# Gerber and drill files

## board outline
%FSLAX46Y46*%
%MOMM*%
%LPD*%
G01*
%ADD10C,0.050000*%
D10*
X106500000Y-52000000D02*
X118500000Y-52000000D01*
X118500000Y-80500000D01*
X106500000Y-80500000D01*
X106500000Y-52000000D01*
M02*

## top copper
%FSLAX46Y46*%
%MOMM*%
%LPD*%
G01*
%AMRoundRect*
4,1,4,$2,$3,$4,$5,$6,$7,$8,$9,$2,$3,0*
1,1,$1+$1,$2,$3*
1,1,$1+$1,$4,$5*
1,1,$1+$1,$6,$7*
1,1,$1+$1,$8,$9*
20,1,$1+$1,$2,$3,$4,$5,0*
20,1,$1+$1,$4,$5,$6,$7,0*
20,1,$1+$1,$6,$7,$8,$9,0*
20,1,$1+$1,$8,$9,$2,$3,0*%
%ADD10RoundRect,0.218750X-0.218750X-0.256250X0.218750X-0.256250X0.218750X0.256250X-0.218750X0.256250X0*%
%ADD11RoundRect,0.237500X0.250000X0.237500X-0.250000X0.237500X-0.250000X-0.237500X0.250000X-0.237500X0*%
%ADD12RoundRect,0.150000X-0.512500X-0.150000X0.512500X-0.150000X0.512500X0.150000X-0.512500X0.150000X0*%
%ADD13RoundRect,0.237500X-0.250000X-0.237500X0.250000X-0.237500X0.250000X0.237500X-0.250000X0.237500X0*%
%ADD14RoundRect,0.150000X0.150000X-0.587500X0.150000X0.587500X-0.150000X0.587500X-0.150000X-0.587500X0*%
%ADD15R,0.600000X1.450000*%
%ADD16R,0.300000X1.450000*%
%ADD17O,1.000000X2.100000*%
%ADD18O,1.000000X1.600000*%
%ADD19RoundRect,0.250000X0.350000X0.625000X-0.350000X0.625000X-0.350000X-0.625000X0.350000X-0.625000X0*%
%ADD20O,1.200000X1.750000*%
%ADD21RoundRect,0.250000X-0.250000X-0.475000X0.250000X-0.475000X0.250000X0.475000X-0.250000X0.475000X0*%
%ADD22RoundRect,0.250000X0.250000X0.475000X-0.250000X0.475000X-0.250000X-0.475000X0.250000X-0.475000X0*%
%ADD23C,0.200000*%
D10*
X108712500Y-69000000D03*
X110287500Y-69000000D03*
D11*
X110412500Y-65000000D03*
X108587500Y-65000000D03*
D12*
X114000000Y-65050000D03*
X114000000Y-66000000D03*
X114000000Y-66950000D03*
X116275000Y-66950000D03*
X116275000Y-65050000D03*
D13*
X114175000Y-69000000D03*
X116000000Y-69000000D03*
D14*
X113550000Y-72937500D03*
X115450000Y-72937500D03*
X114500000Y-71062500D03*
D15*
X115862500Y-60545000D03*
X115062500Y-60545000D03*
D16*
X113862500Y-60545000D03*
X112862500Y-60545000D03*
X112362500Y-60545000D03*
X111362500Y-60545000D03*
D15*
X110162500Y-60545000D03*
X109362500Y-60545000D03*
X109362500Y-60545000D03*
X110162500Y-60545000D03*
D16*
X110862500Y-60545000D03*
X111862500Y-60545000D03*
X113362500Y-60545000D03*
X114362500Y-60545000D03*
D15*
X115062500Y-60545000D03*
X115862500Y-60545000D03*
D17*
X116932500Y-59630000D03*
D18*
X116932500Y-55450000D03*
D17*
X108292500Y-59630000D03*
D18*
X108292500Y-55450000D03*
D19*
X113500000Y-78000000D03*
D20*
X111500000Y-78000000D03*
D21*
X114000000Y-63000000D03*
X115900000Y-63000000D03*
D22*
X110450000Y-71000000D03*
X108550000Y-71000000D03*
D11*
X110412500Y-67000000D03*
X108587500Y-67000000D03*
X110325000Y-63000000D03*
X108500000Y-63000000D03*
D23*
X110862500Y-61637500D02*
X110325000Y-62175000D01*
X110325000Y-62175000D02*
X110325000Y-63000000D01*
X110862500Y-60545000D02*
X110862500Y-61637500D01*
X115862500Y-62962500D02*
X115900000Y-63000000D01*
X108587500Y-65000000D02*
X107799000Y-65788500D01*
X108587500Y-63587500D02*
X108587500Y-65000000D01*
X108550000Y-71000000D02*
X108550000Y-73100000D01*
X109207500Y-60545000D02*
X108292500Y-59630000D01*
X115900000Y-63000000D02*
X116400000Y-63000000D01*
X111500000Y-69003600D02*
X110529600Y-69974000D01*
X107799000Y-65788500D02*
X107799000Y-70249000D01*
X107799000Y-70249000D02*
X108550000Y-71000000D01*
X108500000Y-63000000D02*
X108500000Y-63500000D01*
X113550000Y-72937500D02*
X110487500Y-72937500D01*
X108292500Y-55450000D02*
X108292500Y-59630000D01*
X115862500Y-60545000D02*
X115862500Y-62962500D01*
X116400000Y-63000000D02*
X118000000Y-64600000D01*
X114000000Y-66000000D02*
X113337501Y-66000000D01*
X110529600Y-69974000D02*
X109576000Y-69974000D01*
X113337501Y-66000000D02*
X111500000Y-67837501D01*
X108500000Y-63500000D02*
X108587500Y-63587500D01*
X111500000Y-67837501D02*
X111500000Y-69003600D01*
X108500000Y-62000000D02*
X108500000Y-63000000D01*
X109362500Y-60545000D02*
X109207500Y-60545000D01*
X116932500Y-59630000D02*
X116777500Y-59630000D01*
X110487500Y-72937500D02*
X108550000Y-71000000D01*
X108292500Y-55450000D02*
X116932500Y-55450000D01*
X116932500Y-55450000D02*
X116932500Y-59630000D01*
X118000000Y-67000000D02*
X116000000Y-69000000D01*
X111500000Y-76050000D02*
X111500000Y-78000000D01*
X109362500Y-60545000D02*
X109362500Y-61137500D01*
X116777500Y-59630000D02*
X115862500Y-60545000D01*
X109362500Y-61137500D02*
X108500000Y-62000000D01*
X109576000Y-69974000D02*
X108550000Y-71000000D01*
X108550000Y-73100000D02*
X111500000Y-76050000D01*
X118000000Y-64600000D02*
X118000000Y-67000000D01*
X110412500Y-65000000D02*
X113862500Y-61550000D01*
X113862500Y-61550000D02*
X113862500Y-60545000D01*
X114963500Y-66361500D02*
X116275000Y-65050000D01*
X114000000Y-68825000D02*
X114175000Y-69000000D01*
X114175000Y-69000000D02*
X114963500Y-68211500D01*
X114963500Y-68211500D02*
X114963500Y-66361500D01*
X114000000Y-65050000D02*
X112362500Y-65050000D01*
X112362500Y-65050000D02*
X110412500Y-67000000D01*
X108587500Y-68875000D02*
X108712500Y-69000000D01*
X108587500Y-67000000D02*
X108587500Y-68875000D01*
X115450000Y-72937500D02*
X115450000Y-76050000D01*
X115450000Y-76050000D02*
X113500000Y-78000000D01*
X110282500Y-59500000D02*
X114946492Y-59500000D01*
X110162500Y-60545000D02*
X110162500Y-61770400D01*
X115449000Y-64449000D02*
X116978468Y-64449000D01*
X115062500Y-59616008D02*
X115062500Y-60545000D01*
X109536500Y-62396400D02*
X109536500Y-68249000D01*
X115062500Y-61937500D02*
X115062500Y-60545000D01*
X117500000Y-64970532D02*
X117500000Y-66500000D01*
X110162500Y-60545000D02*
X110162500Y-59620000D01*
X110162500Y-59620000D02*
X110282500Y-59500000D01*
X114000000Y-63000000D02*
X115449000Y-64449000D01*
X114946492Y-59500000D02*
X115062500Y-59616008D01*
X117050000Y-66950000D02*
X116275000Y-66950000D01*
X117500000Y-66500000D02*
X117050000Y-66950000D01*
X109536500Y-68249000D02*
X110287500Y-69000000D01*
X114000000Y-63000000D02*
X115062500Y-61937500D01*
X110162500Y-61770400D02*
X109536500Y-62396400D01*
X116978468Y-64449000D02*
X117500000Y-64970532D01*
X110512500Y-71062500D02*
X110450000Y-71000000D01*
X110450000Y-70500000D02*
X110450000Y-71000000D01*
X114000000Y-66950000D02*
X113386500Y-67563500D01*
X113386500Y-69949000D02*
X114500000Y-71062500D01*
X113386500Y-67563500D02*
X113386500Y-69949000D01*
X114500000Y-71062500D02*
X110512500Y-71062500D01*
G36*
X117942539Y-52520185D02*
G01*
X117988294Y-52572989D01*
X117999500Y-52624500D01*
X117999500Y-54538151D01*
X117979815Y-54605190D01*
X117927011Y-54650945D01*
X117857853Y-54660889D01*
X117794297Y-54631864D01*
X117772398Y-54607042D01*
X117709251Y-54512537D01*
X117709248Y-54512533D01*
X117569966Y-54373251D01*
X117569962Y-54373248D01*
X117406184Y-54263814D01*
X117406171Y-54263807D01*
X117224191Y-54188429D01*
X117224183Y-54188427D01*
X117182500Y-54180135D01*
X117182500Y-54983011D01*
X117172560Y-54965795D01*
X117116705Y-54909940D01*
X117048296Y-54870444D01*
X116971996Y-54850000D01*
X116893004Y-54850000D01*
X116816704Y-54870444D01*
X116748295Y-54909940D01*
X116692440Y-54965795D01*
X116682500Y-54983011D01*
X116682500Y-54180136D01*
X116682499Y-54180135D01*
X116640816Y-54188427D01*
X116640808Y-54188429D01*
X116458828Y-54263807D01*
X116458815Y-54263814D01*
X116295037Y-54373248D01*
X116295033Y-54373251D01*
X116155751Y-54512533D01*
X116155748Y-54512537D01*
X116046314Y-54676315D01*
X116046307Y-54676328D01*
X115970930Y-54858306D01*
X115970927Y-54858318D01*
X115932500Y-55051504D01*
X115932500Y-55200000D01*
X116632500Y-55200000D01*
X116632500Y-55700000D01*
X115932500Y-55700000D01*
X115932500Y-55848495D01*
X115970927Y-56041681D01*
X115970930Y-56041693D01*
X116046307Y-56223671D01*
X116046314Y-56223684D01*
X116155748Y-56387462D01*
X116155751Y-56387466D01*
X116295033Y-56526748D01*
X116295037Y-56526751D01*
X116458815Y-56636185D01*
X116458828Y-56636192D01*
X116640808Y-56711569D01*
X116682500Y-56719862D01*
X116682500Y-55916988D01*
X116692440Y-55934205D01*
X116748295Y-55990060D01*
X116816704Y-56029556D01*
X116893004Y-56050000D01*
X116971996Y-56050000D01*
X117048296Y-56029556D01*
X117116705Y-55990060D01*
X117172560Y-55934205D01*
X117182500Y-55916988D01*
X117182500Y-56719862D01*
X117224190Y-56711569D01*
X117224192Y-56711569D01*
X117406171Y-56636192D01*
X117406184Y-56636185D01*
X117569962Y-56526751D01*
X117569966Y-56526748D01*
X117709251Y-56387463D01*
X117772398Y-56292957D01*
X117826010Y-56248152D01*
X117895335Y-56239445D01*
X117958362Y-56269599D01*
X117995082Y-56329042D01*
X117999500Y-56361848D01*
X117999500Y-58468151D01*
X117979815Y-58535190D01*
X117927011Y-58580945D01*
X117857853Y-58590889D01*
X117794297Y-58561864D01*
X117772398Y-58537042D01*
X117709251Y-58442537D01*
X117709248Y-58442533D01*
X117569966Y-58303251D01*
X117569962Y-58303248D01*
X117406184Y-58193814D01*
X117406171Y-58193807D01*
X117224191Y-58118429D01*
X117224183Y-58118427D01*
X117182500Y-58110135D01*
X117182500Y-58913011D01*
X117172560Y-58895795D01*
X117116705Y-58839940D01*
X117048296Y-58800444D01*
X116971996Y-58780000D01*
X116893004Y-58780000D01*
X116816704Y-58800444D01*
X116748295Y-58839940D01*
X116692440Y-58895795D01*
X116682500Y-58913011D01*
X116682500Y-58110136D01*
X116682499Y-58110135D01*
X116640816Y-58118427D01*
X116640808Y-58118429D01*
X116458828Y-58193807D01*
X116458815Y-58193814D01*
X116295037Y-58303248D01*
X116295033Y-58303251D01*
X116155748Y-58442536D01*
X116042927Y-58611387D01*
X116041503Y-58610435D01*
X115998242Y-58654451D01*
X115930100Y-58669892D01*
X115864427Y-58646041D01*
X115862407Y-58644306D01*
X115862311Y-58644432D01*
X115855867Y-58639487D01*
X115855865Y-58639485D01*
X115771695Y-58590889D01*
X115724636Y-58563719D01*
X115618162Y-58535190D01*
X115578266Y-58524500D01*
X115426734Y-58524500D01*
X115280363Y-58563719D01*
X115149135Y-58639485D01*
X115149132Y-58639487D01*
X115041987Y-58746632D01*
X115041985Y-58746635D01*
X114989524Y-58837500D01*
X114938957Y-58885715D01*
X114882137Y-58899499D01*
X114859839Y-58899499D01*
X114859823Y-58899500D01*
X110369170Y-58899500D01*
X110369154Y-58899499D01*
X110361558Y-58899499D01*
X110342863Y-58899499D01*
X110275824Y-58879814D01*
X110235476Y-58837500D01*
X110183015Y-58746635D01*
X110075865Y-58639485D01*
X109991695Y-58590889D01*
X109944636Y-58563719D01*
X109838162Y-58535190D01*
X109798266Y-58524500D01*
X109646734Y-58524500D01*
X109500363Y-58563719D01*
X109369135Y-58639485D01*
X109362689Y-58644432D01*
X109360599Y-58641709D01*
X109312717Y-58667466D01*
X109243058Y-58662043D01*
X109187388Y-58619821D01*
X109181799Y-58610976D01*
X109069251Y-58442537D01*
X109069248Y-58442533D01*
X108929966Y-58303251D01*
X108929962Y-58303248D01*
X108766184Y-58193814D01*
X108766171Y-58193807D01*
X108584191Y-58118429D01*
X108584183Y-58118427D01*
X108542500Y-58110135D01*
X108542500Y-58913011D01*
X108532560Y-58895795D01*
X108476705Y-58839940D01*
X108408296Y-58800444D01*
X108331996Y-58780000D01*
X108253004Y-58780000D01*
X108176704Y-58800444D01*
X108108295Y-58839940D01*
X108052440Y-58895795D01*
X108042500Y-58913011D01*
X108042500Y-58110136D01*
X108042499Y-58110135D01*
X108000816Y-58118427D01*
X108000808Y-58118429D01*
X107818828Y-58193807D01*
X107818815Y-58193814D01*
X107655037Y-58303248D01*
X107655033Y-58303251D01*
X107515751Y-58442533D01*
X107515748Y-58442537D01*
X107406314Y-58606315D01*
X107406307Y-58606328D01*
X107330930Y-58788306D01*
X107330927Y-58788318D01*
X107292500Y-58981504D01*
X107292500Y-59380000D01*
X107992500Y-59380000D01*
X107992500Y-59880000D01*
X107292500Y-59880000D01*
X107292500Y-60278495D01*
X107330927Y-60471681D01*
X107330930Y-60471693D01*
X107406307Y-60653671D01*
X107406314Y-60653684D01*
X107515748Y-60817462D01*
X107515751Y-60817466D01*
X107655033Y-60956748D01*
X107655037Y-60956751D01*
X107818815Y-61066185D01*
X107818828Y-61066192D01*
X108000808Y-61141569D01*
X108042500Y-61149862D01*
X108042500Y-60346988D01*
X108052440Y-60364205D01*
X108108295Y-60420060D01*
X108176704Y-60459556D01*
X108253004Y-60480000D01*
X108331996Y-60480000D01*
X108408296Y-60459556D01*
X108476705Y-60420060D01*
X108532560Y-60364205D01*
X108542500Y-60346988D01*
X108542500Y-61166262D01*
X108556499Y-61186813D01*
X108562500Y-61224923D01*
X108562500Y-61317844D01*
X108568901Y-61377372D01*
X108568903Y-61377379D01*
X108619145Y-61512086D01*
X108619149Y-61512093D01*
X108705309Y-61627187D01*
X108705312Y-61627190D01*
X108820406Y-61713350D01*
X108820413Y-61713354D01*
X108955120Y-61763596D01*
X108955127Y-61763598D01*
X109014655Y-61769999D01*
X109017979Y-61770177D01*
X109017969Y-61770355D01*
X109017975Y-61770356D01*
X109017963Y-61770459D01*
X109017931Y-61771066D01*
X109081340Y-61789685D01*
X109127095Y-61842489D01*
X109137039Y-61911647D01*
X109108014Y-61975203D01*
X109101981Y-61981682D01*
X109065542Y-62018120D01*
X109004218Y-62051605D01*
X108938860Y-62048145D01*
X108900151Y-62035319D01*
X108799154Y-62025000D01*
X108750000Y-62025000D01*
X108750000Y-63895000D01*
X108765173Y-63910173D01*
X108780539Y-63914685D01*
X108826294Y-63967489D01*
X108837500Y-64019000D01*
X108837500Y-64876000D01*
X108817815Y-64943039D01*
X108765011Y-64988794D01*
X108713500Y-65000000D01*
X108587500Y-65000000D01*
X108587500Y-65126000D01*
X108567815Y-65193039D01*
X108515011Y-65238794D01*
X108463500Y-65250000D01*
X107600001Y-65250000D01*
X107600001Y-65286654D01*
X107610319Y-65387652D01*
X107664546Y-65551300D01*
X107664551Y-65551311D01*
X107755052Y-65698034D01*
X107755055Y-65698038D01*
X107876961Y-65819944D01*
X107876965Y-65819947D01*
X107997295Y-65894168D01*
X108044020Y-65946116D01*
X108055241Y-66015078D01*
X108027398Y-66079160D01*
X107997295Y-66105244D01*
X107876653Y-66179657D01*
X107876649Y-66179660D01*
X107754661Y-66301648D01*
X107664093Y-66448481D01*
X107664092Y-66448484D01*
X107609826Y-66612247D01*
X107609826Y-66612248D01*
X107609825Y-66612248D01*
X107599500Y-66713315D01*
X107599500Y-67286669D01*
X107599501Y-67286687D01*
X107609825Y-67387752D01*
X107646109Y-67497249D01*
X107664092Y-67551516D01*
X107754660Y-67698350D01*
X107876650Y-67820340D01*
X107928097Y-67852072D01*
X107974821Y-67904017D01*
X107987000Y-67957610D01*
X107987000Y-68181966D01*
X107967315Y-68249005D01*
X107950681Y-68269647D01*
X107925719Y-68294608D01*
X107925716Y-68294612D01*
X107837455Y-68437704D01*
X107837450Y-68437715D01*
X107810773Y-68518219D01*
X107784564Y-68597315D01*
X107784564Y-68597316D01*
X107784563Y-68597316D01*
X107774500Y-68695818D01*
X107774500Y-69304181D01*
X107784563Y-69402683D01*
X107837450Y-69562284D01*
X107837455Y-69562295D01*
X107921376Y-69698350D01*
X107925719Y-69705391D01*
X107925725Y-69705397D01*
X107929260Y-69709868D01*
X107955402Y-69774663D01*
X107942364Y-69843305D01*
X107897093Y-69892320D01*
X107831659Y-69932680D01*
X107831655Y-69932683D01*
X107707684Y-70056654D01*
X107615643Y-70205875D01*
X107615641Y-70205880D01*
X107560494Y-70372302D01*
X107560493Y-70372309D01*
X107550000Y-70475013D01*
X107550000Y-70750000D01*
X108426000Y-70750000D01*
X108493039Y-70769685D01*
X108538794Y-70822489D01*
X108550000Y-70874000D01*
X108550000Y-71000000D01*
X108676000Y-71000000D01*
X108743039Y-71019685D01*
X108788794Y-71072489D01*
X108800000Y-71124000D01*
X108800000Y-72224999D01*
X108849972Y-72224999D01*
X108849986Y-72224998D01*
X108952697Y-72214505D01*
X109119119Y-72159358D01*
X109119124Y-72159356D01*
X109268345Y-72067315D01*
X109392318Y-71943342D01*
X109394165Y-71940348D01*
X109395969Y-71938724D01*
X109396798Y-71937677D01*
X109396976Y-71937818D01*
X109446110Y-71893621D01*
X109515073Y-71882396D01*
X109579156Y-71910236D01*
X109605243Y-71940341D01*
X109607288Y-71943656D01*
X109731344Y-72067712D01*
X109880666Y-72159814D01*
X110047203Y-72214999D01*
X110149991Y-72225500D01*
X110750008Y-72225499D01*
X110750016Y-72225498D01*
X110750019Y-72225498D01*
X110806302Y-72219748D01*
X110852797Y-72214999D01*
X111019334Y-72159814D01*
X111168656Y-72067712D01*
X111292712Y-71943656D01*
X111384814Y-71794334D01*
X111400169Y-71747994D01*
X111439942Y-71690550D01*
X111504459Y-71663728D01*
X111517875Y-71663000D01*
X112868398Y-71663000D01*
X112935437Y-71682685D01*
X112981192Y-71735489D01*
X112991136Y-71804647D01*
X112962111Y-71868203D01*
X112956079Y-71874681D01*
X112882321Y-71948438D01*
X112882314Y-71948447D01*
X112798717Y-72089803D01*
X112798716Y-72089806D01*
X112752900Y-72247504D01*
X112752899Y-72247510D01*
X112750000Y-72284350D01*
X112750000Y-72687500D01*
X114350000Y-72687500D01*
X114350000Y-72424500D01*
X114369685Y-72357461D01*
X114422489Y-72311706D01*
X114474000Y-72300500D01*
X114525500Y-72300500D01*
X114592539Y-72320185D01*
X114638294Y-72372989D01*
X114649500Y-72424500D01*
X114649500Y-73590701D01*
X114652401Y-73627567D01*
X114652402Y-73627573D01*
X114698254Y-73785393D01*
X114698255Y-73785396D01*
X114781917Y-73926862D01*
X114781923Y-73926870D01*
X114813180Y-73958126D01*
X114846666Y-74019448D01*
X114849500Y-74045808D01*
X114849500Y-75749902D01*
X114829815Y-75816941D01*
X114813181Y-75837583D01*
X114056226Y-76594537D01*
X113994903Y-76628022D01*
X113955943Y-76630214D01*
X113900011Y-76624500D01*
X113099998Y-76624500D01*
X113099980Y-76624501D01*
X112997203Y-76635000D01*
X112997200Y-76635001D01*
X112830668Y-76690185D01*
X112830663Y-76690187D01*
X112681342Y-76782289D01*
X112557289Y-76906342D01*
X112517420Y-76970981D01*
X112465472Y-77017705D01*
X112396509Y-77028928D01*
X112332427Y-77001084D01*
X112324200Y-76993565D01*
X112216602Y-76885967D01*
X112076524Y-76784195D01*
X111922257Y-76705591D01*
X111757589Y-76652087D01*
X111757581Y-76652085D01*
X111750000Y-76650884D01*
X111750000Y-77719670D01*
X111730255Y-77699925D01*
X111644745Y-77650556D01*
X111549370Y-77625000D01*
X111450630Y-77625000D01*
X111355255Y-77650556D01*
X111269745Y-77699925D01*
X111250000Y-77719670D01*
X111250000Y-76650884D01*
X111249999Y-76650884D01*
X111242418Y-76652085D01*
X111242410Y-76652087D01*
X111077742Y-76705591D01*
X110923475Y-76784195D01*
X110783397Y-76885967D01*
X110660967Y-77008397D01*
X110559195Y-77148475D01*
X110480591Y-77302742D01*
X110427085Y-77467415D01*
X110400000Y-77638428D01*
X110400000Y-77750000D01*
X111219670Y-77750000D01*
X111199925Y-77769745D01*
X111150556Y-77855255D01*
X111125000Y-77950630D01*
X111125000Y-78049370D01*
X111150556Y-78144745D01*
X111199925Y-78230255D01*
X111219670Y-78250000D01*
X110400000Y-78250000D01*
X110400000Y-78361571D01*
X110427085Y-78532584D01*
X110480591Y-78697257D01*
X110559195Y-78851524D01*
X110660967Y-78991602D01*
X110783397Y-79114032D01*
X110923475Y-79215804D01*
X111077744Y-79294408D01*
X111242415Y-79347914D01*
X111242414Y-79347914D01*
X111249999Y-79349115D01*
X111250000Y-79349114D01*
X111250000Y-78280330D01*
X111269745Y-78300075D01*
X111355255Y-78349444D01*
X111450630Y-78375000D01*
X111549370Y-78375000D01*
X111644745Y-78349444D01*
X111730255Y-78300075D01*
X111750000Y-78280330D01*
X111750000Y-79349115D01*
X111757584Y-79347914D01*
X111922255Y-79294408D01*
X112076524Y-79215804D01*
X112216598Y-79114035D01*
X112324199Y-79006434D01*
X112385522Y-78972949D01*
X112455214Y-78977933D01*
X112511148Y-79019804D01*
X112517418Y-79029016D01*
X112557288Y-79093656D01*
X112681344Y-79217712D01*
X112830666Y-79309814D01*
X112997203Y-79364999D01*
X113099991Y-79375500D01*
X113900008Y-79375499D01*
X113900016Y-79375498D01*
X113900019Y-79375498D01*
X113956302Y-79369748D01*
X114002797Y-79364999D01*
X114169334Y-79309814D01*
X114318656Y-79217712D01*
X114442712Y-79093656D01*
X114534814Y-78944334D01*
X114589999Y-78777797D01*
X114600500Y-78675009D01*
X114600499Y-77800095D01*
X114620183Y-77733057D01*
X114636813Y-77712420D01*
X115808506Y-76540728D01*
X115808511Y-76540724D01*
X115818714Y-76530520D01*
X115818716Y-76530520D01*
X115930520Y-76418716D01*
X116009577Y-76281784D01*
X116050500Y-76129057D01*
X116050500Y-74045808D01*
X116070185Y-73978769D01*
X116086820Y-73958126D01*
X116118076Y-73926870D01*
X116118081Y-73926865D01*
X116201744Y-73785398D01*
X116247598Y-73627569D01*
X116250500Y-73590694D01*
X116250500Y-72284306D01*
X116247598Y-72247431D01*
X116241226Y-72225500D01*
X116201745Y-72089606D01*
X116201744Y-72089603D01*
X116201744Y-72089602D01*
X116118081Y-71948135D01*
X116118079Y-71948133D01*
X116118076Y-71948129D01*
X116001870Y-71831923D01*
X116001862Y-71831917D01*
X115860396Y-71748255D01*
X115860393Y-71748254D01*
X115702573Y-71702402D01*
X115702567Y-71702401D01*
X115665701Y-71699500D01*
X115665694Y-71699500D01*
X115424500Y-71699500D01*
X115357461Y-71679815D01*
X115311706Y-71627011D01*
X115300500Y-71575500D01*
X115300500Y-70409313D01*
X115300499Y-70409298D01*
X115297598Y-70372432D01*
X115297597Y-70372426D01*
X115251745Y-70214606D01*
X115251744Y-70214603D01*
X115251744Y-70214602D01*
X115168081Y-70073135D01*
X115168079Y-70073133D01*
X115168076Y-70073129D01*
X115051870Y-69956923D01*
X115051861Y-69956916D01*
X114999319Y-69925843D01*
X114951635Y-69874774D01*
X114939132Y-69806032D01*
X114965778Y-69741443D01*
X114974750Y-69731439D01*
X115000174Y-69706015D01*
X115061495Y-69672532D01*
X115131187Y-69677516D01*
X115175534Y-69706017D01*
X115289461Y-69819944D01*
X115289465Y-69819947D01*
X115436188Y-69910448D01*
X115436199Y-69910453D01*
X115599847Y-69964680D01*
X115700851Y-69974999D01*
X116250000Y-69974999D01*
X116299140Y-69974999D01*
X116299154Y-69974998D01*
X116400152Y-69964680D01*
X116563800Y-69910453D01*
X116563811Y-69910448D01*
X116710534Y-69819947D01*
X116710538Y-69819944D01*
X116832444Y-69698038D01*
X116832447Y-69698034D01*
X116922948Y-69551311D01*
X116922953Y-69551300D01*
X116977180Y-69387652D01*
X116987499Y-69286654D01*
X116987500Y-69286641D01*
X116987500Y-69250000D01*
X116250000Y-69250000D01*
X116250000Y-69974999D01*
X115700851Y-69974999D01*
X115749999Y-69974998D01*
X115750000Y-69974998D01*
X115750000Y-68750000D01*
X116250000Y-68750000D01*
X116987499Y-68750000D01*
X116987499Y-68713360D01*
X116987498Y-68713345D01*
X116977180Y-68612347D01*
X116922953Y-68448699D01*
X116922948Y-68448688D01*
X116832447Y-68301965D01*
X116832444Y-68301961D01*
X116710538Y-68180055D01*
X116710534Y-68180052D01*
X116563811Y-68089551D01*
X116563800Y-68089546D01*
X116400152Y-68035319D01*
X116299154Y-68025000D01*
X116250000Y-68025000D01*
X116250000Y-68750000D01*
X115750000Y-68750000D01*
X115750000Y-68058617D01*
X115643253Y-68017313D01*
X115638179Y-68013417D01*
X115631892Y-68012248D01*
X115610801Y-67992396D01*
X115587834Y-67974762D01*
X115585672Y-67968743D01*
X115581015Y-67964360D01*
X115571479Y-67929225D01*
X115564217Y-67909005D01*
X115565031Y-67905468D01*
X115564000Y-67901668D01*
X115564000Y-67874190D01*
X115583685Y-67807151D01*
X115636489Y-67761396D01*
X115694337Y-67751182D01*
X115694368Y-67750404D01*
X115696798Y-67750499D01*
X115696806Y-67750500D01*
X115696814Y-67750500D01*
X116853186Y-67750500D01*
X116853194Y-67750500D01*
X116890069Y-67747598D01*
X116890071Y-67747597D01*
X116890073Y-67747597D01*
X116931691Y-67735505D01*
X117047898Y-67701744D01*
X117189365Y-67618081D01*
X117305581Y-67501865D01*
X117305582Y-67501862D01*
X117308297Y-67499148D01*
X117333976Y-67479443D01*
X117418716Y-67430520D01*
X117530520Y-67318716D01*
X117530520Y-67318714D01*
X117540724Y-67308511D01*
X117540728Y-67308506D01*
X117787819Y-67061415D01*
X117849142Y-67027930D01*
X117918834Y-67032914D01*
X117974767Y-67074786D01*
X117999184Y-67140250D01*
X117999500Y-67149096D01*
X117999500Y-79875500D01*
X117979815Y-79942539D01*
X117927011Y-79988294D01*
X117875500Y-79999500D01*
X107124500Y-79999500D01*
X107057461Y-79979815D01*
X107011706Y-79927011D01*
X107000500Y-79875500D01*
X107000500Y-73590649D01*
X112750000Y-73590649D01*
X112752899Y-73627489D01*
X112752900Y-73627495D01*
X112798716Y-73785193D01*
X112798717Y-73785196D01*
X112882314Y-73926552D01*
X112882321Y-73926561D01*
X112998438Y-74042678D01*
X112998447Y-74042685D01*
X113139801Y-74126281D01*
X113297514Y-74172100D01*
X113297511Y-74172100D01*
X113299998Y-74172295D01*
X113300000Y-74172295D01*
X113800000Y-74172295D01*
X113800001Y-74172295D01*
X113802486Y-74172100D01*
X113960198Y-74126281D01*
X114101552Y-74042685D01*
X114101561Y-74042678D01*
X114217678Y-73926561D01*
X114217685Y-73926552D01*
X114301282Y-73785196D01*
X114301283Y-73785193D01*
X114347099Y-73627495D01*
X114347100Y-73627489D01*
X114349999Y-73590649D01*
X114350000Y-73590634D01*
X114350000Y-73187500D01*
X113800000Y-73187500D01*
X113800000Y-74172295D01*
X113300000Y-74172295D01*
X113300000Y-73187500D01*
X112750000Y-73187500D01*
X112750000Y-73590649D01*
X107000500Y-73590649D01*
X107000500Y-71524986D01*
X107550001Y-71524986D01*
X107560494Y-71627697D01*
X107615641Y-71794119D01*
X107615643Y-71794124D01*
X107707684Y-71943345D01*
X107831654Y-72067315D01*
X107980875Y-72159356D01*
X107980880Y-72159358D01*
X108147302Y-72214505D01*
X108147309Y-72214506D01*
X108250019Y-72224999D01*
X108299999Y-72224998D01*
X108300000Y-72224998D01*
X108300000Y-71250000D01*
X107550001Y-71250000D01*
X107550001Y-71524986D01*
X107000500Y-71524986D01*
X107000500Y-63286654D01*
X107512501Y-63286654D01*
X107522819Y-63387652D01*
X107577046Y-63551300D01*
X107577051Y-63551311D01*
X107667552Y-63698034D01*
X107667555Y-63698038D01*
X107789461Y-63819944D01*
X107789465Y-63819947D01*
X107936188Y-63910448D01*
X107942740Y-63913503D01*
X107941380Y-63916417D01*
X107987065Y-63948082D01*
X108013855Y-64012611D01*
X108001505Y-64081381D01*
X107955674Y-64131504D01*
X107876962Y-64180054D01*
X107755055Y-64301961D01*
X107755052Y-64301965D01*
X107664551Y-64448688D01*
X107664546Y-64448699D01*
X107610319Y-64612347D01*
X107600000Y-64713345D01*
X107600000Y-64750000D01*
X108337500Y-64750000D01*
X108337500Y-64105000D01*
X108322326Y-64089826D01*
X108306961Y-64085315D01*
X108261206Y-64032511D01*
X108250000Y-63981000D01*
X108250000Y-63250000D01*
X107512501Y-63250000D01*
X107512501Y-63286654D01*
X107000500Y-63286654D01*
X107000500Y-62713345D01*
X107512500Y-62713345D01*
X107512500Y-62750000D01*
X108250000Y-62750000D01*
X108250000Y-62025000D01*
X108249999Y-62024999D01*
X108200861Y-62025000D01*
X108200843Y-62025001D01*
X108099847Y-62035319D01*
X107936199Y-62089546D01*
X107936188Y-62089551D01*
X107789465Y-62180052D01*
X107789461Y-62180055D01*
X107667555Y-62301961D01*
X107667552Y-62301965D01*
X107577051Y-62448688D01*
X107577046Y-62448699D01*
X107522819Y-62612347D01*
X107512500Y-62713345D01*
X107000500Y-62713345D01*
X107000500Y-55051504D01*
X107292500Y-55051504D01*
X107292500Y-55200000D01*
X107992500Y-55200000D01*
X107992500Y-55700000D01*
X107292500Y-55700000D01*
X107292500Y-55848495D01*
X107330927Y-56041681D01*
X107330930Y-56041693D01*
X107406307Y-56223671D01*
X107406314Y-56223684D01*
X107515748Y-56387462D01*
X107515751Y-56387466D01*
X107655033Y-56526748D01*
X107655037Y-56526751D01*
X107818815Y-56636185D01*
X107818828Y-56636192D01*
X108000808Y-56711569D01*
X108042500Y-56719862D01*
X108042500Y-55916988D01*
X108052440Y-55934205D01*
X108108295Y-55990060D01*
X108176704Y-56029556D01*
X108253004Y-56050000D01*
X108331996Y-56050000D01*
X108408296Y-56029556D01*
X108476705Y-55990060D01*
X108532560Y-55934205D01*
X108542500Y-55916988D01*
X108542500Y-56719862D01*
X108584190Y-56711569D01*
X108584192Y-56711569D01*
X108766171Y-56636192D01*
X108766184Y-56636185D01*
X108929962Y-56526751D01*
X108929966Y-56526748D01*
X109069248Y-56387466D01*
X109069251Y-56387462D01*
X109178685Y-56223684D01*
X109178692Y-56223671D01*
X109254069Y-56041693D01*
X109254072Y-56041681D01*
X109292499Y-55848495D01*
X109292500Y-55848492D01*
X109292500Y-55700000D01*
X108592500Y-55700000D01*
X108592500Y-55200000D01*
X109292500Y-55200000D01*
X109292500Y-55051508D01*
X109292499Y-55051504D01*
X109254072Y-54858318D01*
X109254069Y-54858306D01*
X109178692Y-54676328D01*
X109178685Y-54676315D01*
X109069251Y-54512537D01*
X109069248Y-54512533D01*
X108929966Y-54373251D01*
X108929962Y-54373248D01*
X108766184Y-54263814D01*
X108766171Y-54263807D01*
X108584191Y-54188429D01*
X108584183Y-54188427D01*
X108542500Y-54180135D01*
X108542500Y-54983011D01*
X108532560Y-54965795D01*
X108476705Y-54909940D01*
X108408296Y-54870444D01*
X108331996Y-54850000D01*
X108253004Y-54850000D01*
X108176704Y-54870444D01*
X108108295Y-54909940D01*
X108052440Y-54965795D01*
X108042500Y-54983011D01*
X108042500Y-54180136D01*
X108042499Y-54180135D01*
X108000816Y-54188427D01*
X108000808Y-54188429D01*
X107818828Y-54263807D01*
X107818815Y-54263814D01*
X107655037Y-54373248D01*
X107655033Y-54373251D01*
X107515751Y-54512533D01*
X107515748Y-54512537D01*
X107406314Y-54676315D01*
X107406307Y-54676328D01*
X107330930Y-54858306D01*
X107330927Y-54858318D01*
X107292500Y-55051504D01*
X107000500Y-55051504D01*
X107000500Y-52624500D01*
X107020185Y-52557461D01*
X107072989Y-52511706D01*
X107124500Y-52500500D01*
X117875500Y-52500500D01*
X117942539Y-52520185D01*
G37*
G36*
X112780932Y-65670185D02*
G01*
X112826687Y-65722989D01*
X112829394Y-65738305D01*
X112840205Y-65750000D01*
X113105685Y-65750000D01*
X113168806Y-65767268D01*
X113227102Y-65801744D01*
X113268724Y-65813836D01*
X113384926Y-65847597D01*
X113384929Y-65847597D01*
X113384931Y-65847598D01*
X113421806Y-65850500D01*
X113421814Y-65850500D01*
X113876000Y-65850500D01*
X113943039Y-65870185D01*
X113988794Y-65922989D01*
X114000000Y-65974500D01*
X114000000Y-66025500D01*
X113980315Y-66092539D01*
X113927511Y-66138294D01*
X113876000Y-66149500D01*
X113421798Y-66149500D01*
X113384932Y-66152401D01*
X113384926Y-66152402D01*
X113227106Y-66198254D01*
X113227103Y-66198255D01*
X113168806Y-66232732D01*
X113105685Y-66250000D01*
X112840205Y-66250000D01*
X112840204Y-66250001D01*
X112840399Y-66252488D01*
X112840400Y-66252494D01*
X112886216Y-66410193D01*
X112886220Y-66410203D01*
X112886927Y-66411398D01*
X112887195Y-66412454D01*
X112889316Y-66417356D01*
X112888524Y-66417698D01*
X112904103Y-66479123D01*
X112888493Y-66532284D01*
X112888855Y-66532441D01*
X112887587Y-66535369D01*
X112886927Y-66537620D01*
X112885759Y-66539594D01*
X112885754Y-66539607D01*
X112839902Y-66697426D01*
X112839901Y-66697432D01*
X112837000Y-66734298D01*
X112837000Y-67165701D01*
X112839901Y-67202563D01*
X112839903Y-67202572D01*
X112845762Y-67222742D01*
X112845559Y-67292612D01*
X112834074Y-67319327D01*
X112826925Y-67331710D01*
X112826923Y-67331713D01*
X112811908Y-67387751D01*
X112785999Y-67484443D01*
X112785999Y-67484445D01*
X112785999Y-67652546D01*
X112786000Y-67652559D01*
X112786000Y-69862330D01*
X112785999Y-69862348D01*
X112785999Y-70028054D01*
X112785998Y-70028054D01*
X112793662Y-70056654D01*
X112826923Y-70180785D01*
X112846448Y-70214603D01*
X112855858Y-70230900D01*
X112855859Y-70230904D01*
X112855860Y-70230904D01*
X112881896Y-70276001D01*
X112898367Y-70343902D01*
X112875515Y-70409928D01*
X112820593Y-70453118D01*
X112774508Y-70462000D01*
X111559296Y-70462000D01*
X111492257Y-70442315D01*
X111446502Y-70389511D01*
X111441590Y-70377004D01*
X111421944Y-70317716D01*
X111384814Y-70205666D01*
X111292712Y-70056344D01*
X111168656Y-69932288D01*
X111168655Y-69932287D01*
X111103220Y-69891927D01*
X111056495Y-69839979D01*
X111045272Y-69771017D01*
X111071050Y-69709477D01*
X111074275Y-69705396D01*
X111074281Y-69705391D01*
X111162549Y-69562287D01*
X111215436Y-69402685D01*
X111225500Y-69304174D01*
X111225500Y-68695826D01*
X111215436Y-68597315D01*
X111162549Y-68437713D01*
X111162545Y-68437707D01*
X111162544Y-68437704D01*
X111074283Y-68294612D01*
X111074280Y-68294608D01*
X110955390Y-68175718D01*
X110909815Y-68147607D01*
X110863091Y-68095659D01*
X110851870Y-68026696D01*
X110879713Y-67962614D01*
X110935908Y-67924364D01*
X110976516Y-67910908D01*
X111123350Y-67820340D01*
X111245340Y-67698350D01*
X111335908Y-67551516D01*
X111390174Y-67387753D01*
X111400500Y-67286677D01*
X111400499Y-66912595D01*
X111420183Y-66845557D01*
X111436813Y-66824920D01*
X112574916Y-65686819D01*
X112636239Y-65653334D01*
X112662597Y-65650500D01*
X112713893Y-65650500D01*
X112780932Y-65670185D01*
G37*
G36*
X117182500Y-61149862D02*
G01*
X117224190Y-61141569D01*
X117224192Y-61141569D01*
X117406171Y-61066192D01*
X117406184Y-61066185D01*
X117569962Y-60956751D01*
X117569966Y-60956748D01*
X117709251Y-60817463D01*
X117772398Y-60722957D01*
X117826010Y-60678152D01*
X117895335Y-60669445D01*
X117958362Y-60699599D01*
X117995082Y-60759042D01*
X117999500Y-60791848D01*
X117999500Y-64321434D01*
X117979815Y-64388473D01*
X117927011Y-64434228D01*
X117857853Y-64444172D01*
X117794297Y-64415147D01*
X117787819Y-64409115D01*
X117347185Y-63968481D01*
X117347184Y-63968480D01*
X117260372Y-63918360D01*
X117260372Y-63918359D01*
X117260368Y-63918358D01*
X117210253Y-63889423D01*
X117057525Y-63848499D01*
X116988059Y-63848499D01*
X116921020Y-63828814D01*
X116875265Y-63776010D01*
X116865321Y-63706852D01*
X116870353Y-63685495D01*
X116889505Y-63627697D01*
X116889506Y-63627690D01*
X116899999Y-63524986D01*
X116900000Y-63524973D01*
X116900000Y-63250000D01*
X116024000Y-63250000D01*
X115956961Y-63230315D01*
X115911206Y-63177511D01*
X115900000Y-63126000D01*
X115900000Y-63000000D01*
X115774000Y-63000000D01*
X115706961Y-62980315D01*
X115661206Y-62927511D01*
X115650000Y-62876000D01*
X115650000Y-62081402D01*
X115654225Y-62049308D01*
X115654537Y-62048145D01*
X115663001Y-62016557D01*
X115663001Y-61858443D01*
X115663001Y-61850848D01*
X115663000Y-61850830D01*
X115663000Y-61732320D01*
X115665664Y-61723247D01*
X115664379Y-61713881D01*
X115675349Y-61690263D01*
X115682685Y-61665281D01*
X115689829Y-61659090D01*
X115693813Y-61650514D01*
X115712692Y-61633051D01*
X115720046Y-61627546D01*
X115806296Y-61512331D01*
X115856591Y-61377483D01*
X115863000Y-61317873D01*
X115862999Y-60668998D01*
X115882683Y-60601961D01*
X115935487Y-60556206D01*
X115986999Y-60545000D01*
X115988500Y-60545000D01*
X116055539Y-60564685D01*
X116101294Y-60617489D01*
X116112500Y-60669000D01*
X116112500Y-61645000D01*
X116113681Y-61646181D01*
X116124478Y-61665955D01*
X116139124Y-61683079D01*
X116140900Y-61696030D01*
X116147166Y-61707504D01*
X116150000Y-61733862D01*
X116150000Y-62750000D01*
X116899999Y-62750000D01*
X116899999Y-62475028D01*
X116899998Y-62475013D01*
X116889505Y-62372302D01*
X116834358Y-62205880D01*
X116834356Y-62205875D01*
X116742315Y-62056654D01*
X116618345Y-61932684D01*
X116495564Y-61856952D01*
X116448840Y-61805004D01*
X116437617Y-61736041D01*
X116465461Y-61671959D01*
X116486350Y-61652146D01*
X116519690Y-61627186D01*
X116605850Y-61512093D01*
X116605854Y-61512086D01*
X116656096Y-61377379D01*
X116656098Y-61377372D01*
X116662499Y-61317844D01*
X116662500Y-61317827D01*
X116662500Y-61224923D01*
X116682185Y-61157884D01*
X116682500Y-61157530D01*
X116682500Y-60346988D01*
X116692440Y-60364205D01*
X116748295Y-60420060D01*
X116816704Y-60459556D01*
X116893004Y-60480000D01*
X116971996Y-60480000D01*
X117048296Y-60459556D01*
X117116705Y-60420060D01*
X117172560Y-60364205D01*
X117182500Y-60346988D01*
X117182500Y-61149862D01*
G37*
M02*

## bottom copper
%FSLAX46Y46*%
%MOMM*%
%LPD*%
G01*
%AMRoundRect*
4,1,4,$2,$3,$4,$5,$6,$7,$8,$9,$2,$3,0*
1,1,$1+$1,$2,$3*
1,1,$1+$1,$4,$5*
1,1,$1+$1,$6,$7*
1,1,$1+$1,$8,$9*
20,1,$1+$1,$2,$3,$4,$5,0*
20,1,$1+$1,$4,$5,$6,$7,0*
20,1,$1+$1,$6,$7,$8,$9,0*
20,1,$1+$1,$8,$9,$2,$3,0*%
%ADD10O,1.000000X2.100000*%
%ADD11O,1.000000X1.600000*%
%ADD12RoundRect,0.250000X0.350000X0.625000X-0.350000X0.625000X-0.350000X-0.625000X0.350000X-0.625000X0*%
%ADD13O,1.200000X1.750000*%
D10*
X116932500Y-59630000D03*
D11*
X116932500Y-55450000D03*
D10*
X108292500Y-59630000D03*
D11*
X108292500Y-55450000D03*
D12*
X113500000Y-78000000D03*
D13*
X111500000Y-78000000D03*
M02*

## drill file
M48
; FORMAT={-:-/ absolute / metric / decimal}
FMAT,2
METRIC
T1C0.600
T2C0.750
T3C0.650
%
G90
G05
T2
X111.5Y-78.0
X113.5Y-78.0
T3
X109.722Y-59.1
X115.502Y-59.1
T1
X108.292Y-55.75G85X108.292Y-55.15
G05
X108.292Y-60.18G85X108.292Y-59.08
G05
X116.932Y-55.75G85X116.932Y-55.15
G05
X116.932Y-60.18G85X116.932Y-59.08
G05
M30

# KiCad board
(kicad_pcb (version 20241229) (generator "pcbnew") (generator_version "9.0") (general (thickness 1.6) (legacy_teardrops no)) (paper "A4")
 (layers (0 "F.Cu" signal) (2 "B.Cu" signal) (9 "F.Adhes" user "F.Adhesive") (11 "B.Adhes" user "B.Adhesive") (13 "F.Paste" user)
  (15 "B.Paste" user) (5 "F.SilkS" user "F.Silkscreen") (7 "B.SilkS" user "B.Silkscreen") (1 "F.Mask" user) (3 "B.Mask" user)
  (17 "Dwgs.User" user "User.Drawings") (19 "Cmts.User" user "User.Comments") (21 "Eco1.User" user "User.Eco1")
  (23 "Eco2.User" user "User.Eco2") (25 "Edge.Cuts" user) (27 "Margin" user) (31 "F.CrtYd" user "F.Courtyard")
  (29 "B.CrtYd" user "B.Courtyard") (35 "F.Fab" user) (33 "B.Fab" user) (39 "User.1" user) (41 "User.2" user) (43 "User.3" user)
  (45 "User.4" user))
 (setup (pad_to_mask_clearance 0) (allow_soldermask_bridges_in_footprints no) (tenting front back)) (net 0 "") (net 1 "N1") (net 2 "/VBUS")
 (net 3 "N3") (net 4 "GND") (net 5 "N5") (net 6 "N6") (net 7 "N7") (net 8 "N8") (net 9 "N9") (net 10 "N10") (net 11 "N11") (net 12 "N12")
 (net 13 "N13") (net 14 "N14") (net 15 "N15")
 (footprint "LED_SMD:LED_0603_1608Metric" (layer "F.Cu") (at 109.5 69)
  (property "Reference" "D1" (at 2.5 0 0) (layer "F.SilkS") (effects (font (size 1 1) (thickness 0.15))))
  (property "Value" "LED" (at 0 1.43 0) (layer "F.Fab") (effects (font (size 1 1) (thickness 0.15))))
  (pad "1" smd roundrect (at -0.7875 0) (size 0.875 0.95) (layers "F.Cu" "F.Mask" "F.Paste") (roundrect_rratio 0.25) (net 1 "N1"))
  (pad "2" smd roundrect (at 0.7875 0) (size 0.875 0.95) (layers "F.Cu" "F.Mask" "F.Paste") (roundrect_rratio 0.25) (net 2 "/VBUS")))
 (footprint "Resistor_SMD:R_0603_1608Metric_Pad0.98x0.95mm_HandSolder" (layer "F.Cu") (at 109.5 65 180)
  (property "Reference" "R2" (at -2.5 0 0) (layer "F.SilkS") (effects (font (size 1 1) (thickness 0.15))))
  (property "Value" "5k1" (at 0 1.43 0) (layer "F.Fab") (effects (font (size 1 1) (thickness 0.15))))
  (pad "1" smd roundrect (at -0.9125 0 180) (size 0.975 0.95) (layers "F.Cu" "F.Mask" "F.Paste") (roundrect_rratio 0.25) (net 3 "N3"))
  (pad "2" smd roundrect (at 0.9125 0 180) (size 0.975 0.95) (layers "F.Cu" "F.Mask" "F.Paste") (roundrect_rratio 0.25) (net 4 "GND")))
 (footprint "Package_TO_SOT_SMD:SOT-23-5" (layer "F.Cu") (at 115.1375 66)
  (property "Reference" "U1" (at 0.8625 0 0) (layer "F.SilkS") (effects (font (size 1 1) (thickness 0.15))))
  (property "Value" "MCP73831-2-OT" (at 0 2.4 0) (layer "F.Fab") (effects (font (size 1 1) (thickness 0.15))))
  (pad "1" smd roundrect (at -1.1375 -0.95) (size 1.325 0.6) (layers "F.Cu" "F.Mask" "F.Paste") (roundrect_rratio 0.25) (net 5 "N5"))
  (pad "2" smd roundrect (at -1.1375 0) (size 1.325 0.6) (layers "F.Cu" "F.Mask" "F.Paste") (roundrect_rratio 0.25) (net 4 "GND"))
  (pad "3" smd roundrect (at -1.1375 0.95) (size 1.325 0.6) (layers "F.Cu" "F.Mask" "F.Paste") (roundrect_rratio 0.25) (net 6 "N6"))
  (pad "4" smd roundrect (at 1.1375 0.95) (size 1.325 0.6) (layers "F.Cu" "F.Mask" "F.Paste") (roundrect_rratio 0.25) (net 2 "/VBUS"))
  (pad "5" smd roundrect (at 1.1375 -0.95) (size 1.325 0.6) (layers "F.Cu" "F.Mask" "F.Paste") (roundrect_rratio 0.25) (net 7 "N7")))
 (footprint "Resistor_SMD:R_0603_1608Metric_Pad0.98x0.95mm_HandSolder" (layer "F.Cu") (at 115.0875 69)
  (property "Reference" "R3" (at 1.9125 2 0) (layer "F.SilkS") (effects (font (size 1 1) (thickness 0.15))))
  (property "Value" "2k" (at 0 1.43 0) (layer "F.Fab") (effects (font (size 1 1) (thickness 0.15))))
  (pad "1" smd roundrect (at -0.9125 0) (size 0.975 0.95) (layers "F.Cu" "F.Mask" "F.Paste") (roundrect_rratio 0.25) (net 7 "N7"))
  (pad "2" smd roundrect (at 0.9125 0) (size 0.975 0.95) (layers "F.Cu" "F.Mask" "F.Paste") (roundrect_rratio 0.25) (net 4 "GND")))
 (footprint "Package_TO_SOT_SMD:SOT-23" (layer "F.Cu") (at 114.5 72 90)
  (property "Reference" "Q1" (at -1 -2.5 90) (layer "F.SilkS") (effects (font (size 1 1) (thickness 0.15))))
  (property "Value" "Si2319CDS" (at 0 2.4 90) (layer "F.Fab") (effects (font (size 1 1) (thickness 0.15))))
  (pad "1" smd roundrect (at -0.9375 -0.95 90) (size 1.475 0.6) (layers "F.Cu" "F.Mask" "F.Paste") (roundrect_rratio 0.25) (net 4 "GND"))
  (pad "2" smd roundrect (at -0.9375 0.95 90) (size 1.475 0.6) (layers "F.Cu" "F.Mask" "F.Paste") (roundrect_rratio 0.25) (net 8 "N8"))
  (pad "3" smd roundrect (at 0.9375 0 90) (size 1.475 0.6) (layers "F.Cu" "F.Mask" "F.Paste") (roundrect_rratio 0.25) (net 6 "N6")))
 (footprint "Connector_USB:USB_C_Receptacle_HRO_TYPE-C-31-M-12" (layer "F.Cu") (at 112.6125 56.5 180)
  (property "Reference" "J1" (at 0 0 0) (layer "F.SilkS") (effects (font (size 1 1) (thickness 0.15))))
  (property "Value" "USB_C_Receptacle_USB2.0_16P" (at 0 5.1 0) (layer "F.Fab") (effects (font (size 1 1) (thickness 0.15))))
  (pad "" np_thru_hole circle (at -2.89 -2.6 180) (size 0.65 0.65) (drill 0.65) (layers "*.Cu" "*.Mask"))
  (pad "" np_thru_hole circle (at 2.89 -2.6 180) (size 0.65 0.65) (drill 0.65) (layers "*.Cu" "*.Mask"))
  (pad "A1" smd rect (at -3.25 -4.045 180) (size 0.6 1.45) (layers "F.Cu" "F.Mask" "F.Paste") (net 4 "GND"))
  (pad "A4" smd rect (at -2.45 -4.045 180) (size 0.6 1.45) (layers "F.Cu" "F.Mask" "F.Paste") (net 2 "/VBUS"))
  (pad "A5" smd rect (at -1.25 -4.045 180) (size 0.3 1.45) (layers "F.Cu" "F.Mask" "F.Paste") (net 3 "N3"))
  (pad "A6" smd rect (at -0.25 -4.045 180) (size 0.3 1.45) (layers "F.Cu" "F.Mask" "F.Paste") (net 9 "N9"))
  (pad "A7" smd rect (at 0.25 -4.045 180) (size 0.3 1.45) (layers "F.Cu" "F.Mask" "F.Paste") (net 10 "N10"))
  (pad "A8" smd rect (at 1.25 -4.045 180) (size 0.3 1.45) (layers "F.Cu" "F.Mask" "F.Paste") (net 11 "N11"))
  (pad "A9" smd rect (at 2.45 -4.045 180) (size 0.6 1.45) (layers "F.Cu" "F.Mask" "F.Paste") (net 2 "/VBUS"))
  (pad "A12" smd rect (at 3.25 -4.045 180) (size 0.6 1.45) (layers "F.Cu" "F.Mask" "F.Paste") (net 4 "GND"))
  (pad "B1" smd rect (at 3.25 -4.045 180) (size 0.6 1.45) (layers "F.Cu" "F.Mask" "F.Paste") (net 4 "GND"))
  (pad "B4" smd rect (at 2.45 -4.045 180) (size 0.6 1.45) (layers "F.Cu" "F.Mask" "F.Paste") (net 2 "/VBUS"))
  (pad "B5" smd rect (at 1.75 -4.045 180) (size 0.3 1.45) (layers "F.Cu" "F.Mask" "F.Paste") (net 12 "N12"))
  (pad "B6" smd rect (at 0.75 -4.045 180) (size 0.3 1.45) (layers "F.Cu" "F.Mask" "F.Paste") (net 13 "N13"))
  (pad "B7" smd rect (at -0.75 -4.045 180) (size 0.3 1.45) (layers "F.Cu" "F.Mask" "F.Paste") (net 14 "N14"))
  (pad "B8" smd rect (at -1.75 -4.045 180) (size 0.3 1.45) (layers "F.Cu" "F.Mask" "F.Paste") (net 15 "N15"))
  (pad "B9" smd rect (at -2.45 -4.045 180) (size 0.6 1.45) (layers "F.Cu" "F.Mask" "F.Paste") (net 2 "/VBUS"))
  (pad "B12" smd rect (at -3.25 -4.045 180) (size 0.6 1.45) (layers "F.Cu" "F.Mask" "F.Paste") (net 4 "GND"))
  (pad "S1" thru_hole oval (at -4.32 -3.13 180) (size 1 2.1) (drill oval 0.6 1.7) (layers "*.Cu" "*.Mask") (remove_unused_layers no)
   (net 4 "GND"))
  (pad "S1" thru_hole oval (at -4.32 1.05 180) (size 1 1.6) (drill oval 0.6 1.2) (layers "*.Cu" "*.Mask") (remove_unused_layers no)
   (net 4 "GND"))
  (pad "S1" thru_hole oval (at 4.32 -3.13 180) (size 1 2.1) (drill oval 0.6 1.7) (layers "*.Cu" "*.Mask") (remove_unused_layers no)
   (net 4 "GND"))
  (pad "S1" thru_hole oval (at 4.32 1.05 180) (size 1 1.6) (drill oval 0.6 1.2) (layers "*.Cu" "*.Mask") (remove_unused_layers no)
   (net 4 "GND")))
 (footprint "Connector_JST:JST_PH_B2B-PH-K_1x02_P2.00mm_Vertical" (layer "F.Cu") (at 113.5 78 180)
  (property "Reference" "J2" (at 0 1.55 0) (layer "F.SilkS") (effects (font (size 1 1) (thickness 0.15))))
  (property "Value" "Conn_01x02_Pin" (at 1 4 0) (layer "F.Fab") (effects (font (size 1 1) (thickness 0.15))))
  (pad "1" thru_hole roundrect (at 0 0 180) (size 1.2 1.75) (drill 0.75) (layers "*.Cu" "*.Mask") (remove_unused_layers no)
   (roundrect_rratio 0.208333) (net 8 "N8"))
  (pad "2" thru_hole oval (at 2 0 180) (size 1.2 1.75) (drill 0.75) (layers "*.Cu" "*.Mask") (remove_unused_layers no) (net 4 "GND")))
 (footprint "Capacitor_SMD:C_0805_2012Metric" (layer "F.Cu") (at 114.95 63)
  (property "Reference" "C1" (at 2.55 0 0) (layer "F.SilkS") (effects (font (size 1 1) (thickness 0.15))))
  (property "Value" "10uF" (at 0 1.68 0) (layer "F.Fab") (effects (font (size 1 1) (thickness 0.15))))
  (pad "1" smd roundrect (at -0.95 0) (size 1 1.45) (layers "F.Cu" "F.Mask" "F.Paste") (roundrect_rratio 0.25) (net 2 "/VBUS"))
  (pad "2" smd roundrect (at 0.95 0) (size 1 1.45) (layers "F.Cu" "F.Mask" "F.Paste") (roundrect_rratio 0.25) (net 4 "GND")))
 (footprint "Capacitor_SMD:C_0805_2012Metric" (layer "F.Cu") (at 109.5 71 180)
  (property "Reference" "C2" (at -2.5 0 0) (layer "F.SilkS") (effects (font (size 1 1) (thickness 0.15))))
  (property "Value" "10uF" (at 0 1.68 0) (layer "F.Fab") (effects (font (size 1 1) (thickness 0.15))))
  (pad "1" smd roundrect (at -0.95 0 180) (size 1 1.45) (layers "F.Cu" "F.Mask" "F.Paste") (roundrect_rratio 0.25) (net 6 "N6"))
  (pad "2" smd roundrect (at 0.95 0 180) (size 1 1.45) (layers "F.Cu" "F.Mask" "F.Paste") (roundrect_rratio 0.25) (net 4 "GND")))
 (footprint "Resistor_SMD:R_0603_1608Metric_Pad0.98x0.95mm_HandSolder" (layer "F.Cu") (at 109.5 67 180)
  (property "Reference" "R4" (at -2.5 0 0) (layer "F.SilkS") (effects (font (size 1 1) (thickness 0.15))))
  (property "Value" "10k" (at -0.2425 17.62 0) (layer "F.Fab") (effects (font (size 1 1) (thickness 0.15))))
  (pad "1" smd roundrect (at -0.9125 0 180) (size 0.975 0.95) (layers "F.Cu" "F.Mask" "F.Paste") (roundrect_rratio 0.25) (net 5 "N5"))
  (pad "2" smd roundrect (at 0.9125 0 180) (size 0.975 0.95) (layers "F.Cu" "F.Mask" "F.Paste") (roundrect_rratio 0.25) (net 1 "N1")))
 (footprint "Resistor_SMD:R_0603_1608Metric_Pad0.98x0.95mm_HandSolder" (layer "F.Cu") (at 109.4125 63 180)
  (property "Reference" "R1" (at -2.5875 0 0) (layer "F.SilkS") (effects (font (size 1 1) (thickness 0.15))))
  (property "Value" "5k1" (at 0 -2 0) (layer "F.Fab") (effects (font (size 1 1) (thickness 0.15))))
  (pad "1" smd roundrect (at -0.9125 0 180) (size 0.975 0.95) (layers "F.Cu" "F.Mask" "F.Paste") (roundrect_rratio 0.25) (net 12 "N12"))
  (pad "2" smd roundrect (at 0.9125 0 180) (size 0.975 0.95) (layers "F.Cu" "F.Mask" "F.Paste") (roundrect_rratio 0.25) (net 4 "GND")))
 (gr_rect (start 106.5 52) (end 118.5 80.5) (stroke (width 0.05) (type default)) (fill no) (layer "Edge.Cuts"))
 (segment (start 110.8625 61.6375) (end 110.325 62.175) (width 0.2) (layer "F.Cu") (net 12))
 (segment (start 110.325 62.175) (end 110.325 63) (width 0.2) (layer "F.Cu") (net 12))
 (segment (start 110.8625 60.545) (end 110.8625 61.6375) (width 0.2) (layer "F.Cu") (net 12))
 (segment (start 115.8625 62.9625) (end 115.9 63) (width 0.2) (layer "F.Cu") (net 4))
 (segment (start 108.5875 65) (end 107.799 65.7885) (width 0.2) (layer "F.Cu") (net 4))
 (segment (start 108.5875 63.5875) (end 108.5875 65) (width 0.2) (layer "F.Cu") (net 4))
 (segment (start 108.55 71) (end 108.55 73.1) (width 0.2) (layer "F.Cu") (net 4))
 (segment (start 109.2075 60.545) (end 108.2925 59.63) (width 0.2) (layer "F.Cu") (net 4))
 (segment (start 115.9 63) (end 116.4 63) (width 0.2) (layer "F.Cu") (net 4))
 (segment (start 111.5 69.0036) (end 110.5296 69.974) (width 0.2) (layer "F.Cu") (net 4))
 (segment (start 107.799 65.7885) (end 107.799 70.249) (width 0.2) (layer "F.Cu") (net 4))
 (segment (start 107.799 70.249) (end 108.55 71) (width 0.2) (layer "F.Cu") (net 4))
 (segment (start 108.5 63) (end 108.5 63.5) (width 0.2) (layer "F.Cu") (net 4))
 (segment (start 113.55 72.9375) (end 110.4875 72.9375) (width 0.2) (layer "F.Cu") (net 4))
 (segment (start 108.2925 55.45) (end 108.2925 59.63) (width 0.2) (layer "F.Cu") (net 4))
 (segment (start 115.8625 60.545) (end 115.8625 62.9625) (width 0.2) (layer "F.Cu") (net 4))
 (segment (start 116.4 63) (end 118 64.6) (width 0.2) (layer "F.Cu") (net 4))
 (segment (start 114 66) (end 113.337501 66) (width 0.2) (layer "F.Cu") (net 4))
 (segment (start 110.5296 69.974) (end 109.576 69.974) (width 0.2) (layer "F.Cu") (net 4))
 (segment (start 113.337501 66) (end 111.5 67.837501) (width 0.2) (layer "F.Cu") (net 4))
 (segment (start 108.5 63.5) (end 108.5875 63.5875) (width 0.2) (layer "F.Cu") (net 4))
 (segment (start 111.5 67.837501) (end 111.5 69.0036) (width 0.2) (layer "F.Cu") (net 4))
 (segment (start 108.5 62) (end 108.5 63) (width 0.2) (layer "F.Cu") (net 4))
 (segment (start 109.3625 60.545) (end 109.2075 60.545) (width 0.2) (layer "F.Cu") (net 4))
 (segment (start 116.9325 59.63) (end 116.7775 59.63) (width 0.2) (layer "F.Cu") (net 4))
 (segment (start 110.4875 72.9375) (end 108.55 71) (width 0.2) (layer "F.Cu") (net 4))
 (segment (start 108.2925 55.45) (end 116.9325 55.45) (width 0.2) (layer "F.Cu") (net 4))
 (segment (start 116.9325 55.45) (end 116.9325 59.63) (width 0.2) (layer "F.Cu") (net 4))
 (segment (start 118 67) (end 116 69) (width 0.2) (layer "F.Cu") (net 4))
 (segment (start 111.5 76.05) (end 111.5 78) (width 0.2) (layer "F.Cu") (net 4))
 (segment (start 109.3625 60.545) (end 109.3625 61.1375) (width 0.2) (layer "F.Cu") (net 4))
 (segment (start 116.7775 59.63) (end 115.8625 60.545) (width 0.2) (layer "F.Cu") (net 4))
 (segment (start 109.3625 61.1375) (end 108.5 62) (width 0.2) (layer "F.Cu") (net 4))
 (segment (start 109.576 69.974) (end 108.55 71) (width 0.2) (layer "F.Cu") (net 4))
 (segment (start 108.55 73.1) (end 111.5 76.05) (width 0.2) (layer "F.Cu") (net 4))
 (segment (start 118 64.6) (end 118 67) (width 0.2) (layer "F.Cu") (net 4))
 (segment (start 110.4125 65) (end 113.8625 61.55) (width 0.2) (layer "F.Cu") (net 3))
 (segment (start 113.8625 61.55) (end 113.8625 60.545) (width 0.2) (layer "F.Cu") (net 3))
 (segment (start 114.9635 66.3615) (end 116.275 65.05) (width 0.2) (layer "F.Cu") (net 7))
 (segment (start 114 68.825) (end 114.175 69) (width 0.2) (layer "F.Cu") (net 7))
 (segment (start 114.175 69) (end 114.9635 68.2115) (width 0.2) (layer "F.Cu") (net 7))
 (segment (start 114.9635 68.2115) (end 114.9635 66.3615) (width 0.2) (layer "F.Cu") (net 7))
 (segment (start 114 65.05) (end 112.3625 65.05) (width 0.2) (layer "F.Cu") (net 5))
 (segment (start 112.3625 65.05) (end 110.4125 67) (width 0.2) (layer "F.Cu") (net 5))
 (segment (start 108.5875 68.875) (end 108.7125 69) (width 0.2) (layer "F.Cu") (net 1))
 (segment (start 108.5875 67) (end 108.5875 68.875) (width 0.2) (layer "F.Cu") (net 1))
 (segment (start 115.45 72.9375) (end 115.45 76.05) (width 0.2) (layer "F.Cu") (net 8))
 (segment (start 115.45 76.05) (end 113.5 78) (width 0.2) (layer "F.Cu") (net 8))
 (segment (start 110.2825 59.5) (end 114.946492 59.5) (width 0.2) (layer "F.Cu") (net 2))
 (segment (start 110.1625 60.545) (end 110.1625 61.7704) (width 0.2) (layer "F.Cu") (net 2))
 (segment (start 115.449 64.449) (end 116.978468 64.449) (width 0.2) (layer "F.Cu") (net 2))
 (segment (start 115.0625 59.616008) (end 115.0625 60.545) (width 0.2) (layer "F.Cu") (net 2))
 (segment (start 109.5365 62.3964) (end 109.5365 68.249) (width 0.2) (layer "F.Cu") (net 2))
 (segment (start 115.0625 61.9375) (end 115.0625 60.545) (width 0.2) (layer "F.Cu") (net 2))
 (segment (start 117.5 64.970532) (end 117.5 66.5) (width 0.2) (layer "F.Cu") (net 2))
 (segment (start 110.1625 60.545) (end 110.1625 59.62) (width 0.2) (layer "F.Cu") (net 2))
 (segment (start 110.1625 59.62) (end 110.2825 59.5) (width 0.2) (layer "F.Cu") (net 2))
 (segment (start 114 63) (end 115.449 64.449) (width 0.2) (layer "F.Cu") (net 2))
 (segment (start 114.946492 59.5) (end 115.0625 59.616008) (width 0.2) (layer "F.Cu") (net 2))
 (segment (start 117.05 66.95) (end 116.275 66.95) (width 0.2) (layer "F.Cu") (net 2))
 (segment (start 117.5 66.5) (end 117.05 66.95) (width 0.2) (layer "F.Cu") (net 2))
 (segment (start 109.5365 68.249) (end 110.2875 69) (width 0.2) (layer "F.Cu") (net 2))
 (segment (start 114 63) (end 115.0625 61.9375) (width 0.2) (layer "F.Cu") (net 2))
 (segment (start 110.1625 61.7704) (end 109.5365 62.3964) (width 0.2) (layer "F.Cu") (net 2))
 (segment (start 116.978468 64.449) (end 117.5 64.970532) (width 0.2) (layer "F.Cu") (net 2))
 (segment (start 110.5125 71.0625) (end 110.45 71) (width 0.2) (layer "F.Cu") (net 6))
 (segment (start 110.45 70.5) (end 110.45 71) (width 0.2) (layer "F.Cu") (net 6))
 (segment (start 114 66.95) (end 113.3865 67.5635) (width 0.2) (layer "F.Cu") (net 6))
 (segment (start 113.3865 69.949) (end 114.5 71.0625) (width 0.2) (layer "F.Cu") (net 6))
 (segment (start 113.3865 67.5635) (end 113.3865 69.949) (width 0.2) (layer "F.Cu") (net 6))
 (segment (start 114.5 71.0625) (end 110.5125 71.0625) (width 0.2) (layer "F.Cu") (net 6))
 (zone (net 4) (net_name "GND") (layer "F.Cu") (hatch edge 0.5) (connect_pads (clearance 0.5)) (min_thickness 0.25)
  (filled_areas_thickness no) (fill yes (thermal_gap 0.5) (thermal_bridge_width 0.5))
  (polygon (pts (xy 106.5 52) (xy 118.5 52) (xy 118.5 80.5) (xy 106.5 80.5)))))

